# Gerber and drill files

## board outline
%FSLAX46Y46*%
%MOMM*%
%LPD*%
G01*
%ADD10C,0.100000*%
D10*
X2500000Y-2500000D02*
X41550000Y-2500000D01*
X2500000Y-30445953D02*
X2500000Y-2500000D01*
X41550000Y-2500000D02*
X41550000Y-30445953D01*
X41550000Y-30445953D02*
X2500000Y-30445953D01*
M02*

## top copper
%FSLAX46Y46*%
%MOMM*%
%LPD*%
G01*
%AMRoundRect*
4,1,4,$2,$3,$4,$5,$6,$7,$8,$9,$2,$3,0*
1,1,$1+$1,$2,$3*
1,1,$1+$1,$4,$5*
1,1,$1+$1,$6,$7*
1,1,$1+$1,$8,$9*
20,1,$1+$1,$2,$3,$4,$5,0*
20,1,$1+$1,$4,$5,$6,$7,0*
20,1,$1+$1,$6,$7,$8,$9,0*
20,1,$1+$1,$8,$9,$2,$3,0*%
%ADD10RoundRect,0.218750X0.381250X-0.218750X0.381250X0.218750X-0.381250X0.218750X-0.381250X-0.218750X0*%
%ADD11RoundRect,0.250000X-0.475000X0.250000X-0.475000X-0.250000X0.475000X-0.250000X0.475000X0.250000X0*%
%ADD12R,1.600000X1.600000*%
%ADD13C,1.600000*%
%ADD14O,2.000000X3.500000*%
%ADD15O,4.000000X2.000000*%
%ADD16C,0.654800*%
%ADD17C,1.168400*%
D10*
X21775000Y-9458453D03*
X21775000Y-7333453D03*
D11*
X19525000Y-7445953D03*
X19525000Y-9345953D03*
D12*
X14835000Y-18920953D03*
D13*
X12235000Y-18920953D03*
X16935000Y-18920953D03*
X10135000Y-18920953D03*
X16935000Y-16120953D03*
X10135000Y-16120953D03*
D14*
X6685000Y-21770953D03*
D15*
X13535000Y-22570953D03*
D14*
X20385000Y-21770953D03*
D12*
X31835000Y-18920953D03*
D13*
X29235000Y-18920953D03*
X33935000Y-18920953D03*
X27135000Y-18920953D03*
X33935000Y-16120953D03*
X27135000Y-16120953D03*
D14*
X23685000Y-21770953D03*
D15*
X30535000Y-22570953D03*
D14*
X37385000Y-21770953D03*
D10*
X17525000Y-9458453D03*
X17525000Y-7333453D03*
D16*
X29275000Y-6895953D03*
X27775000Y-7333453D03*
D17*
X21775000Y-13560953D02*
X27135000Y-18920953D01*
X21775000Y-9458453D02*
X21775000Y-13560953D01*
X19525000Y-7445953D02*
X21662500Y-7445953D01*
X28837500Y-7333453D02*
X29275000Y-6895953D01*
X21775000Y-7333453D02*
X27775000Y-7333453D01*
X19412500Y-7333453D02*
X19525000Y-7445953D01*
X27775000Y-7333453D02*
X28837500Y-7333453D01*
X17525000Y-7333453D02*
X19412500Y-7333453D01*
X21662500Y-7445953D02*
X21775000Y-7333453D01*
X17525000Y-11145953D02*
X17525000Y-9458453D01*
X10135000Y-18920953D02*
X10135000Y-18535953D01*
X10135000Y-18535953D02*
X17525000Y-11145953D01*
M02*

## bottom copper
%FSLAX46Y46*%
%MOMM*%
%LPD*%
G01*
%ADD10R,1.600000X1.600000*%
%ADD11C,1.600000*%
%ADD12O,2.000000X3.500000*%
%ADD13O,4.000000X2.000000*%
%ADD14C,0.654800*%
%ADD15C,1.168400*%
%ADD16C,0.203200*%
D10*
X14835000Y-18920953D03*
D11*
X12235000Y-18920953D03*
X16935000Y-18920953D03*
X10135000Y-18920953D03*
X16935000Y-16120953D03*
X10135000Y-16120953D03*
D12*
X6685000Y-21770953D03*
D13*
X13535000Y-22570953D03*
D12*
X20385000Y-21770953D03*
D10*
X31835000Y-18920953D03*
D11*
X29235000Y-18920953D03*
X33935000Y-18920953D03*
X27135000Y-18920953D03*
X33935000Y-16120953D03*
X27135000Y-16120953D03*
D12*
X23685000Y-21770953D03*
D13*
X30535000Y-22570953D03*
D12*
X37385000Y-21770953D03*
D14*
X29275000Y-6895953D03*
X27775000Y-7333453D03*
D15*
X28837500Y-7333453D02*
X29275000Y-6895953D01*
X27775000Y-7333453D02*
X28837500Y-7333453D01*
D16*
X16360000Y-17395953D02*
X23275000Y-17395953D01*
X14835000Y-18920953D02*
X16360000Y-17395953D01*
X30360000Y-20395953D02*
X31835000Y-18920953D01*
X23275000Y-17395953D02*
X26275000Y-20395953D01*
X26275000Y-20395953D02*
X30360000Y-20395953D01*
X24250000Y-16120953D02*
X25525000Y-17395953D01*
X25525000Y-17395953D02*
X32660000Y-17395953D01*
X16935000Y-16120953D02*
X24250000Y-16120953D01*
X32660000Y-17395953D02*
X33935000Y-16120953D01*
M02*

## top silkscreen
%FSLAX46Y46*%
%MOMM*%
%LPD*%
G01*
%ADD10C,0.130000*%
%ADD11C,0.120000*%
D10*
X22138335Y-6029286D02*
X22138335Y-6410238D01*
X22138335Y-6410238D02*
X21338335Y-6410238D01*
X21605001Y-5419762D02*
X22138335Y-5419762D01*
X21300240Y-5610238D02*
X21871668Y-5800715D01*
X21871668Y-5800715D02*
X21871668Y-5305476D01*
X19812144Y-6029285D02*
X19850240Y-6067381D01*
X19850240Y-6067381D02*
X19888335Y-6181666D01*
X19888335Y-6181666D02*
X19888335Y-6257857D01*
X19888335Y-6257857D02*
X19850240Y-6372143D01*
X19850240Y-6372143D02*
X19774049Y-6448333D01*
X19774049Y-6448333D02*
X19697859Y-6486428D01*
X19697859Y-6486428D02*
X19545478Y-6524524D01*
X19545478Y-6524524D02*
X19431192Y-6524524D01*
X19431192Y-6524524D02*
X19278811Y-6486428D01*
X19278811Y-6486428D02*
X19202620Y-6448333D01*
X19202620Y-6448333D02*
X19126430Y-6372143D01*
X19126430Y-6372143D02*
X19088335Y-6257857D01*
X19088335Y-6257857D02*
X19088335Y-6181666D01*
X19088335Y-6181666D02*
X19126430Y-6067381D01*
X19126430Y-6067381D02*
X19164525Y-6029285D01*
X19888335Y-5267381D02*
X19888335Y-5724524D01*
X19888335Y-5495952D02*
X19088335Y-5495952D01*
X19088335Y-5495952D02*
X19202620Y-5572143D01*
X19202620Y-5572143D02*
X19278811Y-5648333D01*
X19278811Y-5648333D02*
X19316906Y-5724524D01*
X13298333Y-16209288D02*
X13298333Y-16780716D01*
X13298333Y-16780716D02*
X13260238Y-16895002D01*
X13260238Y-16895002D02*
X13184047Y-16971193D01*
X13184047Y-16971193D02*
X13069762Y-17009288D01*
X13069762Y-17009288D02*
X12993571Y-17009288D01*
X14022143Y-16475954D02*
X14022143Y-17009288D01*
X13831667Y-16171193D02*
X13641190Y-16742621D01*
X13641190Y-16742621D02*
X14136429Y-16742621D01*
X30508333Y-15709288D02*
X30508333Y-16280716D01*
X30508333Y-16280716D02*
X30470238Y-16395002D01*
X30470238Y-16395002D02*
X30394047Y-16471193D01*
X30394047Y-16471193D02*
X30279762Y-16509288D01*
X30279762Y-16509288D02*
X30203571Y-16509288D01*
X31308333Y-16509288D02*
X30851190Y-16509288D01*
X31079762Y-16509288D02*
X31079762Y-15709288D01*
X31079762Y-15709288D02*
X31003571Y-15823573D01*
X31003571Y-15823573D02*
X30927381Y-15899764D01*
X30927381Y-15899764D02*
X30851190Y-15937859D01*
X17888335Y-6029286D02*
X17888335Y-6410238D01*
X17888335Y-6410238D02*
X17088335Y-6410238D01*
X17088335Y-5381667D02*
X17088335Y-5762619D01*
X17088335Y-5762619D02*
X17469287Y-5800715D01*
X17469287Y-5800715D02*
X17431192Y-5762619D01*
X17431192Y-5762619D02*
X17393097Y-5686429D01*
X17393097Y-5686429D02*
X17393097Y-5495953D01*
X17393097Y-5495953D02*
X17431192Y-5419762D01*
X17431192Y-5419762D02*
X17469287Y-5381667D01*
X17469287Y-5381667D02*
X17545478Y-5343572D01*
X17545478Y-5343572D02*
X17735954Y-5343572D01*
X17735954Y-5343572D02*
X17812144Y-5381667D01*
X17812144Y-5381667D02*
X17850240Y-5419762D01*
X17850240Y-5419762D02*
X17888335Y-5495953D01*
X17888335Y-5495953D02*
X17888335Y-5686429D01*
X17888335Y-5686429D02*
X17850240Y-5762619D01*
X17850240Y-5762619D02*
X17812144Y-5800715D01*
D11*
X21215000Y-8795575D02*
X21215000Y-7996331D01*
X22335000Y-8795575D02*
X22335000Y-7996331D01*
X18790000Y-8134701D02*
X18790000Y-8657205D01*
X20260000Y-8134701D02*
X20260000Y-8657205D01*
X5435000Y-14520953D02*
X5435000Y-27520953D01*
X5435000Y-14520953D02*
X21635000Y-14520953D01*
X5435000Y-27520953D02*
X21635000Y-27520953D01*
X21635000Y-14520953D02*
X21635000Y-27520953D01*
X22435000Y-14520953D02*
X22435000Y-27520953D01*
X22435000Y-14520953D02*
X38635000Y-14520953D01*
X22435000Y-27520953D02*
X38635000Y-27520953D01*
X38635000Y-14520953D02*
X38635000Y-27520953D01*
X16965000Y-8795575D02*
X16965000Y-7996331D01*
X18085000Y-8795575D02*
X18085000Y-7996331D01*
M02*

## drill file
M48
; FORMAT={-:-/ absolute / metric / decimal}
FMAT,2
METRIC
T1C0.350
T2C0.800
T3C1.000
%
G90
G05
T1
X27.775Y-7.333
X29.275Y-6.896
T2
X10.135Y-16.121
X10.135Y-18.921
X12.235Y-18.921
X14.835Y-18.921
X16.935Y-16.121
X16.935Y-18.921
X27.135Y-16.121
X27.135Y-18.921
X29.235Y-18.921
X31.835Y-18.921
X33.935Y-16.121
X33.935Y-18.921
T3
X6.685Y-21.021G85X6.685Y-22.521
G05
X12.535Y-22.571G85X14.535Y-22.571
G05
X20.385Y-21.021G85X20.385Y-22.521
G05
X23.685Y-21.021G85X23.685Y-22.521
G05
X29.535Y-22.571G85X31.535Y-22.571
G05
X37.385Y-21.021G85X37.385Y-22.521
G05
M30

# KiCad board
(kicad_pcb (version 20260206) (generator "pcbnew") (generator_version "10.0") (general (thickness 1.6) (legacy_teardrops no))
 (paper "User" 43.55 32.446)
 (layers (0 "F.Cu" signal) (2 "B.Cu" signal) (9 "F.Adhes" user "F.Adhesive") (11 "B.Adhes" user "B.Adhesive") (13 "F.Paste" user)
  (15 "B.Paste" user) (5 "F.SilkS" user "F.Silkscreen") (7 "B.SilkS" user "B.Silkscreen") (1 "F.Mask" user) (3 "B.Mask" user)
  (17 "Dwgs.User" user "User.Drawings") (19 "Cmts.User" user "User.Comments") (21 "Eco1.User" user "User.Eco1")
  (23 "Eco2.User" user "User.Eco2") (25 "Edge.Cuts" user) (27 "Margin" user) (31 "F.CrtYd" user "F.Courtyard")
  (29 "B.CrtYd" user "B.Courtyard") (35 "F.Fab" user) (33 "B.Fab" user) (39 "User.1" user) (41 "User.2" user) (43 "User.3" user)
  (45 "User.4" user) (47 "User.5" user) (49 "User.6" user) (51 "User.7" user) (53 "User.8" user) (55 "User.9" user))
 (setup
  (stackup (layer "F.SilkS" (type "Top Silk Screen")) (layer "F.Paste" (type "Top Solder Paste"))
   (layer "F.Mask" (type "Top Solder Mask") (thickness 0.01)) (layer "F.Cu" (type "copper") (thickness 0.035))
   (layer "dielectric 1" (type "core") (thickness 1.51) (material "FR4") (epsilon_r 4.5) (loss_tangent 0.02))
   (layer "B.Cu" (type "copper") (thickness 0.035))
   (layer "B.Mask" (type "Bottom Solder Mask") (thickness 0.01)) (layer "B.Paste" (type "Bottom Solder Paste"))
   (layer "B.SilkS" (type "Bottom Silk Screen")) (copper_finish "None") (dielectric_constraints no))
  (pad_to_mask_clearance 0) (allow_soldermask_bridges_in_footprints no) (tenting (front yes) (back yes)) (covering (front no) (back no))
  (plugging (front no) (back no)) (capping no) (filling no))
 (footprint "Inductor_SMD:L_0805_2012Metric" (layer "F.Cu") (at 21.775 8.395953 90)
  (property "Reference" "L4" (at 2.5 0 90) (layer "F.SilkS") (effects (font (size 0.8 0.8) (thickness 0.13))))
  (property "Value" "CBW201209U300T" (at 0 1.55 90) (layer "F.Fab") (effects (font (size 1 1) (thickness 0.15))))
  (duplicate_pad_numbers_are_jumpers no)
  (fp_line (start -0.399622 -0.56) (end 0.399622 -0.56) (stroke (width 0.12) (type solid)) (layer "F.SilkS"))
  (fp_line (start -0.399622 0.56) (end 0.399622 0.56) (stroke (width 0.12) (type solid)) (layer "F.SilkS"))
  (pad "1" smd roundrect (at -1.0625 0 90) (size 0.875 1.2) (layers "F.Cu" "F.Mask" "F.Paste") (roundrect_rratio 0.25) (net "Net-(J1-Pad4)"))
  (pad "2" smd roundrect (at 1.0625 0 90) (size 0.875 1.2) (layers "F.Cu" "F.Mask" "F.Paste") (roundrect_rratio 0.25) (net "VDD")))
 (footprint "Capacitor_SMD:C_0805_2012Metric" (layer "F.Cu") (at 19.525 8.395953 -90)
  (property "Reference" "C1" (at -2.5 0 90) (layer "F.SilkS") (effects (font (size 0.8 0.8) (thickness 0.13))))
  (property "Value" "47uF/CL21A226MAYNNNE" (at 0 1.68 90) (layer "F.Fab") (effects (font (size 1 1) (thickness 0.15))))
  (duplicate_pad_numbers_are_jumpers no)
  (fp_line (start -0.261252 0.735) (end 0.261252 0.735) (stroke (width 0.12) (type solid)) (layer "F.SilkS"))
  (fp_line (start -0.261252 -0.735) (end 0.261252 -0.735) (stroke (width 0.12) (type solid)) (layer "F.SilkS"))
  (pad "1" smd roundrect (at -0.95 0 270) (size 1 1.45) (layers "F.Cu" "F.Mask" "F.Paste") (roundrect_rratio 0.25) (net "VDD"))
  (pad "2" smd roundrect (at 0.95 0 270) (size 1 1.45) (layers "F.Cu" "F.Mask" "F.Paste") (roundrect_rratio 0.25) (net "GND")))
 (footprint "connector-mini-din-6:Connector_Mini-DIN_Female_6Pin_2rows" (layer "F.Cu") (at 14.835 18.920953)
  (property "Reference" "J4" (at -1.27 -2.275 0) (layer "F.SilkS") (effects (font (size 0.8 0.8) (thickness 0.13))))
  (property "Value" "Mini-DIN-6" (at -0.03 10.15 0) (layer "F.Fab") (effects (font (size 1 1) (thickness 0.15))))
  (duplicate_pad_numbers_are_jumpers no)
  (fp_line (start -9.4 -4.4) (end -9.4 8.6) (stroke (width 0.12) (type solid)) (layer "F.SilkS"))
  (fp_line (start -9.4 -4.4) (end 6.8 -4.4) (stroke (width 0.12) (type solid)) (layer "F.SilkS"))
  (fp_line (start -9.4 8.6) (end 6.8 8.6) (stroke (width 0.12) (type solid)) (layer "F.SilkS"))
  (fp_line (start 6.8 -4.4) (end 6.8 8.6) (stroke (width 0.12) (type solid)) (layer "F.SilkS"))
  (pad "1" thru_hole rect (at 0 0) (size 1.6 1.6) (drill 0.8) (layers "*.Cu" "*.Mask") (remove_unused_layers no) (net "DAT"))
  (pad "2" thru_hole circle (at -2.6 0) (size 1.6 1.6) (drill 0.8) (layers "*.Cu" "*.Mask") (remove_unused_layers no)
   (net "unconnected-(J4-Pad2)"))
  (pad "3" thru_hole circle (at 2.1 0) (size 1.6 1.6) (drill 0.8) (layers "*.Cu" "*.Mask") (remove_unused_layers no) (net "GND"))
  (pad "4" thru_hole circle (at -4.7 0) (size 1.6 1.6) (drill 0.8) (layers "*.Cu" "*.Mask") (remove_unused_layers no) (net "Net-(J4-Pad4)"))
  (pad "5" thru_hole circle (at 2.1 -2.8) (size 1.6 1.6) (drill 0.8) (layers "*.Cu" "*.Mask") (remove_unused_layers no) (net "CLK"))
  (pad "6" thru_hole circle (at -4.7 -2.8) (size 1.6 1.6) (drill 0.8) (layers "*.Cu" "*.Mask") (remove_unused_layers no)
   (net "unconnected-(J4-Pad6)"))
  (pad "7" thru_hole oval (at -8.15 2.85) (size 2 3.5) (drill oval 1 2.5) (layers "*.Cu" "*.Mask") (remove_unused_layers no))
  (pad "7" thru_hole oval (at -1.3 3.65) (size 4 2) (drill oval 3 1) (layers "*.Cu" "*.Mask") (remove_unused_layers no))
  (pad "7" thru_hole oval (at 5.55 2.85) (size 2 3.5) (drill oval 1 2.5) (layers "*.Cu" "*.Mask") (remove_unused_layers no)))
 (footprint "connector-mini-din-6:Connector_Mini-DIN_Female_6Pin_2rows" (layer "F.Cu") (at 31.835 18.920953)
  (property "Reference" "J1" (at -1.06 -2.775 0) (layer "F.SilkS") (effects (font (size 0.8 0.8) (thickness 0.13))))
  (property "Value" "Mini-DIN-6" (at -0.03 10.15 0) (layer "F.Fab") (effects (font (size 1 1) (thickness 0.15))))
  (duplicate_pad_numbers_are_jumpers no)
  (fp_line (start -9.4 -4.4) (end -9.4 8.6) (stroke (width 0.12) (type solid)) (layer "F.SilkS"))
  (fp_line (start -9.4 -4.4) (end 6.8 -4.4) (stroke (width 0.12) (type solid)) (layer "F.SilkS"))
  (fp_line (start -9.4 8.6) (end 6.8 8.6) (stroke (width 0.12) (type solid)) (layer "F.SilkS"))
  (fp_line (start 6.8 -4.4) (end 6.8 8.6) (stroke (width 0.12) (type solid)) (layer "F.SilkS"))
  (pad "1" thru_hole rect (at 0 0) (size 1.6 1.6) (drill 0.8) (layers "*.Cu" "*.Mask") (remove_unused_layers no) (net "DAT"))
  (pad "2" thru_hole circle (at -2.6 0) (size 1.6 1.6) (drill 0.8) (layers "*.Cu" "*.Mask") (remove_unused_layers no)
   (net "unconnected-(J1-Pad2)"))
  (pad "3" thru_hole circle (at 2.1 0) (size 1.6 1.6) (drill 0.8) (layers "*.Cu" "*.Mask") (remove_unused_layers no) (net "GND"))
  (pad "4" thru_hole circle (at -4.7 0) (size 1.6 1.6) (drill 0.8) (layers "*.Cu" "*.Mask") (remove_unused_layers no) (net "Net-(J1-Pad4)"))
  (pad "5" thru_hole circle (at 2.1 -2.8) (size 1.6 1.6) (drill 0.8) (layers "*.Cu" "*.Mask") (remove_unused_layers no) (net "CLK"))
  (pad "6" thru_hole circle (at -4.7 -2.8) (size 1.6 1.6) (drill 0.8) (layers "*.Cu" "*.Mask") (remove_unused_layers no)
   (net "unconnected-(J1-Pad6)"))
  (pad "7" thru_hole oval (at -8.15 2.85) (size 2 3.5) (drill oval 1 2.5) (layers "*.Cu" "*.Mask") (remove_unused_layers no))
  (pad "7" thru_hole oval (at -1.3 3.65) (size 4 2) (drill oval 3 1) (layers "*.Cu" "*.Mask") (remove_unused_layers no))
  (pad "7" thru_hole oval (at 5.55 2.85) (size 2 3.5) (drill oval 1 2.5) (layers "*.Cu" "*.Mask") (remove_unused_layers no)))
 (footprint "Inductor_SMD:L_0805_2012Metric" (layer "F.Cu") (at 17.525 8.395953 90)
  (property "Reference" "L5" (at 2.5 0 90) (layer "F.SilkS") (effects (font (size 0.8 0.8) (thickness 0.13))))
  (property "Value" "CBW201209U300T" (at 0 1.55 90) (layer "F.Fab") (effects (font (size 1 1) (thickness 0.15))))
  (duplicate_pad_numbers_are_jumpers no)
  (fp_line (start -0.399622 -0.56) (end 0.399622 -0.56) (stroke (width 0.12) (type solid)) (layer "F.SilkS"))
  (fp_line (start -0.399622 0.56) (end 0.399622 0.56) (stroke (width 0.12) (type solid)) (layer "F.SilkS"))
  (pad "1" smd roundrect (at -1.0625 0 90) (size 0.875 1.2) (layers "F.Cu" "F.Mask" "F.Paste") (roundrect_rratio 0.25) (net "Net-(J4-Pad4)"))
  (pad "2" smd roundrect (at 1.0625 0 90) (size 0.875 1.2) (layers "F.Cu" "F.Mask" "F.Paste") (roundrect_rratio 0.25) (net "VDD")))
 (gr_line (start 2.5 2.5) (end 41.55 2.5) (stroke (width 0.1) (type default)) (layer "Edge.Cuts"))
 (gr_line (start 2.5 30.445953) (end 2.5 2.5) (stroke (width 0.1) (type default)) (layer "Edge.Cuts"))
 (gr_line (start 41.55 2.5) (end 41.55 30.445953) (stroke (width 0.1) (type default)) (layer "Edge.Cuts"))
 (gr_line (start 41.55 30.445953) (end 2.5 30.445953) (stroke (width 0.1) (type default)) (layer "Edge.Cuts"))
 (segment (start 21.775 13.560953) (end 27.135 18.920953) (width 1.1684) (layer "F.Cu") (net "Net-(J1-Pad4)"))
 (segment (start 21.775 9.458453) (end 21.775 13.560953) (width 1.1684) (layer "F.Cu") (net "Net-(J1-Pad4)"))
 (segment (start 19.525 7.445953) (end 21.6625 7.445953) (width 1.1684) (layer "F.Cu") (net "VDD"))
 (segment (start 28.8375 7.333453) (end 29.275 6.895953) (width 1.1684) (layer "F.Cu") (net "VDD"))
 (segment (start 21.775 7.333453) (end 27.775 7.333453) (width 1.1684) (layer "F.Cu") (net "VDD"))
 (segment (start 19.4125 7.333453) (end 19.525 7.445953) (width 1.1684) (layer "F.Cu") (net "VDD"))
 (segment (start 27.775 7.333453) (end 28.8375 7.333453) (width 1.1684) (layer "F.Cu") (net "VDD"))
 (segment (start 17.525 7.333453) (end 19.4125 7.333453) (width 1.1684) (layer "F.Cu") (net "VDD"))
 (segment (start 21.6625 7.445953) (end 21.775 7.333453) (width 1.1684) (layer "F.Cu") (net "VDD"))
 (via (at 29.275 6.895953) (size 0.6548) (drill 0.35) (layers "F.Cu" "B.Cu") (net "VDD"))
 (via (at 27.775 7.333453) (size 0.6548) (drill 0.35) (layers "F.Cu" "B.Cu") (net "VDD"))
 (segment (start 28.8375 7.333453) (end 29.275 6.895953) (width 1.1684) (layer "B.Cu") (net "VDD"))
 (segment (start 27.775 7.333453) (end 28.8375 7.333453) (width 1.1684) (layer "B.Cu") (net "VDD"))
 (segment (start 16.36 17.395953) (end 23.275 17.395953) (width 0.2032) (layer "B.Cu") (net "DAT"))
 (segment (start 14.835 18.920953) (end 16.36 17.395953) (width 0.2032) (layer "B.Cu") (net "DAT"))
 (segment (start 30.36 20.395953) (end 31.835 18.920953) (width 0.2032) (layer "B.Cu") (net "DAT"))
 (segment (start 23.275 17.395953) (end 26.275 20.395953) (width 0.2032) (layer "B.Cu") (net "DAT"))
 (segment (start 26.275 20.395953) (end 30.36 20.395953) (width 0.2032) (layer "B.Cu") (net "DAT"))
 (segment (start 17.525 11.145953) (end 17.525 9.458453) (width 1.1684) (layer "F.Cu") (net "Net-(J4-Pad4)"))
 (segment (start 10.135 18.920953) (end 10.135 18.535953) (width 1.1684) (layer "F.Cu") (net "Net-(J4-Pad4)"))
 (segment (start 10.135 18.535953) (end 17.525 11.145953) (width 1.1684) (layer "F.Cu") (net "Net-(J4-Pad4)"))
 (segment (start 24.25 16.120953) (end 25.525 17.395953) (width 0.2032) (layer "B.Cu") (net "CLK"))
 (segment (start 25.525 17.395953) (end 32.66 17.395953) (width 0.2032) (layer "B.Cu") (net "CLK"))
 (segment (start 16.935 16.120953) (end 24.25 16.120953) (width 0.2032) (layer "B.Cu") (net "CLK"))
 (segment (start 32.66 17.395953) (end 33.935 16.120953) (width 0.2032) (layer "B.Cu") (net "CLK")))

